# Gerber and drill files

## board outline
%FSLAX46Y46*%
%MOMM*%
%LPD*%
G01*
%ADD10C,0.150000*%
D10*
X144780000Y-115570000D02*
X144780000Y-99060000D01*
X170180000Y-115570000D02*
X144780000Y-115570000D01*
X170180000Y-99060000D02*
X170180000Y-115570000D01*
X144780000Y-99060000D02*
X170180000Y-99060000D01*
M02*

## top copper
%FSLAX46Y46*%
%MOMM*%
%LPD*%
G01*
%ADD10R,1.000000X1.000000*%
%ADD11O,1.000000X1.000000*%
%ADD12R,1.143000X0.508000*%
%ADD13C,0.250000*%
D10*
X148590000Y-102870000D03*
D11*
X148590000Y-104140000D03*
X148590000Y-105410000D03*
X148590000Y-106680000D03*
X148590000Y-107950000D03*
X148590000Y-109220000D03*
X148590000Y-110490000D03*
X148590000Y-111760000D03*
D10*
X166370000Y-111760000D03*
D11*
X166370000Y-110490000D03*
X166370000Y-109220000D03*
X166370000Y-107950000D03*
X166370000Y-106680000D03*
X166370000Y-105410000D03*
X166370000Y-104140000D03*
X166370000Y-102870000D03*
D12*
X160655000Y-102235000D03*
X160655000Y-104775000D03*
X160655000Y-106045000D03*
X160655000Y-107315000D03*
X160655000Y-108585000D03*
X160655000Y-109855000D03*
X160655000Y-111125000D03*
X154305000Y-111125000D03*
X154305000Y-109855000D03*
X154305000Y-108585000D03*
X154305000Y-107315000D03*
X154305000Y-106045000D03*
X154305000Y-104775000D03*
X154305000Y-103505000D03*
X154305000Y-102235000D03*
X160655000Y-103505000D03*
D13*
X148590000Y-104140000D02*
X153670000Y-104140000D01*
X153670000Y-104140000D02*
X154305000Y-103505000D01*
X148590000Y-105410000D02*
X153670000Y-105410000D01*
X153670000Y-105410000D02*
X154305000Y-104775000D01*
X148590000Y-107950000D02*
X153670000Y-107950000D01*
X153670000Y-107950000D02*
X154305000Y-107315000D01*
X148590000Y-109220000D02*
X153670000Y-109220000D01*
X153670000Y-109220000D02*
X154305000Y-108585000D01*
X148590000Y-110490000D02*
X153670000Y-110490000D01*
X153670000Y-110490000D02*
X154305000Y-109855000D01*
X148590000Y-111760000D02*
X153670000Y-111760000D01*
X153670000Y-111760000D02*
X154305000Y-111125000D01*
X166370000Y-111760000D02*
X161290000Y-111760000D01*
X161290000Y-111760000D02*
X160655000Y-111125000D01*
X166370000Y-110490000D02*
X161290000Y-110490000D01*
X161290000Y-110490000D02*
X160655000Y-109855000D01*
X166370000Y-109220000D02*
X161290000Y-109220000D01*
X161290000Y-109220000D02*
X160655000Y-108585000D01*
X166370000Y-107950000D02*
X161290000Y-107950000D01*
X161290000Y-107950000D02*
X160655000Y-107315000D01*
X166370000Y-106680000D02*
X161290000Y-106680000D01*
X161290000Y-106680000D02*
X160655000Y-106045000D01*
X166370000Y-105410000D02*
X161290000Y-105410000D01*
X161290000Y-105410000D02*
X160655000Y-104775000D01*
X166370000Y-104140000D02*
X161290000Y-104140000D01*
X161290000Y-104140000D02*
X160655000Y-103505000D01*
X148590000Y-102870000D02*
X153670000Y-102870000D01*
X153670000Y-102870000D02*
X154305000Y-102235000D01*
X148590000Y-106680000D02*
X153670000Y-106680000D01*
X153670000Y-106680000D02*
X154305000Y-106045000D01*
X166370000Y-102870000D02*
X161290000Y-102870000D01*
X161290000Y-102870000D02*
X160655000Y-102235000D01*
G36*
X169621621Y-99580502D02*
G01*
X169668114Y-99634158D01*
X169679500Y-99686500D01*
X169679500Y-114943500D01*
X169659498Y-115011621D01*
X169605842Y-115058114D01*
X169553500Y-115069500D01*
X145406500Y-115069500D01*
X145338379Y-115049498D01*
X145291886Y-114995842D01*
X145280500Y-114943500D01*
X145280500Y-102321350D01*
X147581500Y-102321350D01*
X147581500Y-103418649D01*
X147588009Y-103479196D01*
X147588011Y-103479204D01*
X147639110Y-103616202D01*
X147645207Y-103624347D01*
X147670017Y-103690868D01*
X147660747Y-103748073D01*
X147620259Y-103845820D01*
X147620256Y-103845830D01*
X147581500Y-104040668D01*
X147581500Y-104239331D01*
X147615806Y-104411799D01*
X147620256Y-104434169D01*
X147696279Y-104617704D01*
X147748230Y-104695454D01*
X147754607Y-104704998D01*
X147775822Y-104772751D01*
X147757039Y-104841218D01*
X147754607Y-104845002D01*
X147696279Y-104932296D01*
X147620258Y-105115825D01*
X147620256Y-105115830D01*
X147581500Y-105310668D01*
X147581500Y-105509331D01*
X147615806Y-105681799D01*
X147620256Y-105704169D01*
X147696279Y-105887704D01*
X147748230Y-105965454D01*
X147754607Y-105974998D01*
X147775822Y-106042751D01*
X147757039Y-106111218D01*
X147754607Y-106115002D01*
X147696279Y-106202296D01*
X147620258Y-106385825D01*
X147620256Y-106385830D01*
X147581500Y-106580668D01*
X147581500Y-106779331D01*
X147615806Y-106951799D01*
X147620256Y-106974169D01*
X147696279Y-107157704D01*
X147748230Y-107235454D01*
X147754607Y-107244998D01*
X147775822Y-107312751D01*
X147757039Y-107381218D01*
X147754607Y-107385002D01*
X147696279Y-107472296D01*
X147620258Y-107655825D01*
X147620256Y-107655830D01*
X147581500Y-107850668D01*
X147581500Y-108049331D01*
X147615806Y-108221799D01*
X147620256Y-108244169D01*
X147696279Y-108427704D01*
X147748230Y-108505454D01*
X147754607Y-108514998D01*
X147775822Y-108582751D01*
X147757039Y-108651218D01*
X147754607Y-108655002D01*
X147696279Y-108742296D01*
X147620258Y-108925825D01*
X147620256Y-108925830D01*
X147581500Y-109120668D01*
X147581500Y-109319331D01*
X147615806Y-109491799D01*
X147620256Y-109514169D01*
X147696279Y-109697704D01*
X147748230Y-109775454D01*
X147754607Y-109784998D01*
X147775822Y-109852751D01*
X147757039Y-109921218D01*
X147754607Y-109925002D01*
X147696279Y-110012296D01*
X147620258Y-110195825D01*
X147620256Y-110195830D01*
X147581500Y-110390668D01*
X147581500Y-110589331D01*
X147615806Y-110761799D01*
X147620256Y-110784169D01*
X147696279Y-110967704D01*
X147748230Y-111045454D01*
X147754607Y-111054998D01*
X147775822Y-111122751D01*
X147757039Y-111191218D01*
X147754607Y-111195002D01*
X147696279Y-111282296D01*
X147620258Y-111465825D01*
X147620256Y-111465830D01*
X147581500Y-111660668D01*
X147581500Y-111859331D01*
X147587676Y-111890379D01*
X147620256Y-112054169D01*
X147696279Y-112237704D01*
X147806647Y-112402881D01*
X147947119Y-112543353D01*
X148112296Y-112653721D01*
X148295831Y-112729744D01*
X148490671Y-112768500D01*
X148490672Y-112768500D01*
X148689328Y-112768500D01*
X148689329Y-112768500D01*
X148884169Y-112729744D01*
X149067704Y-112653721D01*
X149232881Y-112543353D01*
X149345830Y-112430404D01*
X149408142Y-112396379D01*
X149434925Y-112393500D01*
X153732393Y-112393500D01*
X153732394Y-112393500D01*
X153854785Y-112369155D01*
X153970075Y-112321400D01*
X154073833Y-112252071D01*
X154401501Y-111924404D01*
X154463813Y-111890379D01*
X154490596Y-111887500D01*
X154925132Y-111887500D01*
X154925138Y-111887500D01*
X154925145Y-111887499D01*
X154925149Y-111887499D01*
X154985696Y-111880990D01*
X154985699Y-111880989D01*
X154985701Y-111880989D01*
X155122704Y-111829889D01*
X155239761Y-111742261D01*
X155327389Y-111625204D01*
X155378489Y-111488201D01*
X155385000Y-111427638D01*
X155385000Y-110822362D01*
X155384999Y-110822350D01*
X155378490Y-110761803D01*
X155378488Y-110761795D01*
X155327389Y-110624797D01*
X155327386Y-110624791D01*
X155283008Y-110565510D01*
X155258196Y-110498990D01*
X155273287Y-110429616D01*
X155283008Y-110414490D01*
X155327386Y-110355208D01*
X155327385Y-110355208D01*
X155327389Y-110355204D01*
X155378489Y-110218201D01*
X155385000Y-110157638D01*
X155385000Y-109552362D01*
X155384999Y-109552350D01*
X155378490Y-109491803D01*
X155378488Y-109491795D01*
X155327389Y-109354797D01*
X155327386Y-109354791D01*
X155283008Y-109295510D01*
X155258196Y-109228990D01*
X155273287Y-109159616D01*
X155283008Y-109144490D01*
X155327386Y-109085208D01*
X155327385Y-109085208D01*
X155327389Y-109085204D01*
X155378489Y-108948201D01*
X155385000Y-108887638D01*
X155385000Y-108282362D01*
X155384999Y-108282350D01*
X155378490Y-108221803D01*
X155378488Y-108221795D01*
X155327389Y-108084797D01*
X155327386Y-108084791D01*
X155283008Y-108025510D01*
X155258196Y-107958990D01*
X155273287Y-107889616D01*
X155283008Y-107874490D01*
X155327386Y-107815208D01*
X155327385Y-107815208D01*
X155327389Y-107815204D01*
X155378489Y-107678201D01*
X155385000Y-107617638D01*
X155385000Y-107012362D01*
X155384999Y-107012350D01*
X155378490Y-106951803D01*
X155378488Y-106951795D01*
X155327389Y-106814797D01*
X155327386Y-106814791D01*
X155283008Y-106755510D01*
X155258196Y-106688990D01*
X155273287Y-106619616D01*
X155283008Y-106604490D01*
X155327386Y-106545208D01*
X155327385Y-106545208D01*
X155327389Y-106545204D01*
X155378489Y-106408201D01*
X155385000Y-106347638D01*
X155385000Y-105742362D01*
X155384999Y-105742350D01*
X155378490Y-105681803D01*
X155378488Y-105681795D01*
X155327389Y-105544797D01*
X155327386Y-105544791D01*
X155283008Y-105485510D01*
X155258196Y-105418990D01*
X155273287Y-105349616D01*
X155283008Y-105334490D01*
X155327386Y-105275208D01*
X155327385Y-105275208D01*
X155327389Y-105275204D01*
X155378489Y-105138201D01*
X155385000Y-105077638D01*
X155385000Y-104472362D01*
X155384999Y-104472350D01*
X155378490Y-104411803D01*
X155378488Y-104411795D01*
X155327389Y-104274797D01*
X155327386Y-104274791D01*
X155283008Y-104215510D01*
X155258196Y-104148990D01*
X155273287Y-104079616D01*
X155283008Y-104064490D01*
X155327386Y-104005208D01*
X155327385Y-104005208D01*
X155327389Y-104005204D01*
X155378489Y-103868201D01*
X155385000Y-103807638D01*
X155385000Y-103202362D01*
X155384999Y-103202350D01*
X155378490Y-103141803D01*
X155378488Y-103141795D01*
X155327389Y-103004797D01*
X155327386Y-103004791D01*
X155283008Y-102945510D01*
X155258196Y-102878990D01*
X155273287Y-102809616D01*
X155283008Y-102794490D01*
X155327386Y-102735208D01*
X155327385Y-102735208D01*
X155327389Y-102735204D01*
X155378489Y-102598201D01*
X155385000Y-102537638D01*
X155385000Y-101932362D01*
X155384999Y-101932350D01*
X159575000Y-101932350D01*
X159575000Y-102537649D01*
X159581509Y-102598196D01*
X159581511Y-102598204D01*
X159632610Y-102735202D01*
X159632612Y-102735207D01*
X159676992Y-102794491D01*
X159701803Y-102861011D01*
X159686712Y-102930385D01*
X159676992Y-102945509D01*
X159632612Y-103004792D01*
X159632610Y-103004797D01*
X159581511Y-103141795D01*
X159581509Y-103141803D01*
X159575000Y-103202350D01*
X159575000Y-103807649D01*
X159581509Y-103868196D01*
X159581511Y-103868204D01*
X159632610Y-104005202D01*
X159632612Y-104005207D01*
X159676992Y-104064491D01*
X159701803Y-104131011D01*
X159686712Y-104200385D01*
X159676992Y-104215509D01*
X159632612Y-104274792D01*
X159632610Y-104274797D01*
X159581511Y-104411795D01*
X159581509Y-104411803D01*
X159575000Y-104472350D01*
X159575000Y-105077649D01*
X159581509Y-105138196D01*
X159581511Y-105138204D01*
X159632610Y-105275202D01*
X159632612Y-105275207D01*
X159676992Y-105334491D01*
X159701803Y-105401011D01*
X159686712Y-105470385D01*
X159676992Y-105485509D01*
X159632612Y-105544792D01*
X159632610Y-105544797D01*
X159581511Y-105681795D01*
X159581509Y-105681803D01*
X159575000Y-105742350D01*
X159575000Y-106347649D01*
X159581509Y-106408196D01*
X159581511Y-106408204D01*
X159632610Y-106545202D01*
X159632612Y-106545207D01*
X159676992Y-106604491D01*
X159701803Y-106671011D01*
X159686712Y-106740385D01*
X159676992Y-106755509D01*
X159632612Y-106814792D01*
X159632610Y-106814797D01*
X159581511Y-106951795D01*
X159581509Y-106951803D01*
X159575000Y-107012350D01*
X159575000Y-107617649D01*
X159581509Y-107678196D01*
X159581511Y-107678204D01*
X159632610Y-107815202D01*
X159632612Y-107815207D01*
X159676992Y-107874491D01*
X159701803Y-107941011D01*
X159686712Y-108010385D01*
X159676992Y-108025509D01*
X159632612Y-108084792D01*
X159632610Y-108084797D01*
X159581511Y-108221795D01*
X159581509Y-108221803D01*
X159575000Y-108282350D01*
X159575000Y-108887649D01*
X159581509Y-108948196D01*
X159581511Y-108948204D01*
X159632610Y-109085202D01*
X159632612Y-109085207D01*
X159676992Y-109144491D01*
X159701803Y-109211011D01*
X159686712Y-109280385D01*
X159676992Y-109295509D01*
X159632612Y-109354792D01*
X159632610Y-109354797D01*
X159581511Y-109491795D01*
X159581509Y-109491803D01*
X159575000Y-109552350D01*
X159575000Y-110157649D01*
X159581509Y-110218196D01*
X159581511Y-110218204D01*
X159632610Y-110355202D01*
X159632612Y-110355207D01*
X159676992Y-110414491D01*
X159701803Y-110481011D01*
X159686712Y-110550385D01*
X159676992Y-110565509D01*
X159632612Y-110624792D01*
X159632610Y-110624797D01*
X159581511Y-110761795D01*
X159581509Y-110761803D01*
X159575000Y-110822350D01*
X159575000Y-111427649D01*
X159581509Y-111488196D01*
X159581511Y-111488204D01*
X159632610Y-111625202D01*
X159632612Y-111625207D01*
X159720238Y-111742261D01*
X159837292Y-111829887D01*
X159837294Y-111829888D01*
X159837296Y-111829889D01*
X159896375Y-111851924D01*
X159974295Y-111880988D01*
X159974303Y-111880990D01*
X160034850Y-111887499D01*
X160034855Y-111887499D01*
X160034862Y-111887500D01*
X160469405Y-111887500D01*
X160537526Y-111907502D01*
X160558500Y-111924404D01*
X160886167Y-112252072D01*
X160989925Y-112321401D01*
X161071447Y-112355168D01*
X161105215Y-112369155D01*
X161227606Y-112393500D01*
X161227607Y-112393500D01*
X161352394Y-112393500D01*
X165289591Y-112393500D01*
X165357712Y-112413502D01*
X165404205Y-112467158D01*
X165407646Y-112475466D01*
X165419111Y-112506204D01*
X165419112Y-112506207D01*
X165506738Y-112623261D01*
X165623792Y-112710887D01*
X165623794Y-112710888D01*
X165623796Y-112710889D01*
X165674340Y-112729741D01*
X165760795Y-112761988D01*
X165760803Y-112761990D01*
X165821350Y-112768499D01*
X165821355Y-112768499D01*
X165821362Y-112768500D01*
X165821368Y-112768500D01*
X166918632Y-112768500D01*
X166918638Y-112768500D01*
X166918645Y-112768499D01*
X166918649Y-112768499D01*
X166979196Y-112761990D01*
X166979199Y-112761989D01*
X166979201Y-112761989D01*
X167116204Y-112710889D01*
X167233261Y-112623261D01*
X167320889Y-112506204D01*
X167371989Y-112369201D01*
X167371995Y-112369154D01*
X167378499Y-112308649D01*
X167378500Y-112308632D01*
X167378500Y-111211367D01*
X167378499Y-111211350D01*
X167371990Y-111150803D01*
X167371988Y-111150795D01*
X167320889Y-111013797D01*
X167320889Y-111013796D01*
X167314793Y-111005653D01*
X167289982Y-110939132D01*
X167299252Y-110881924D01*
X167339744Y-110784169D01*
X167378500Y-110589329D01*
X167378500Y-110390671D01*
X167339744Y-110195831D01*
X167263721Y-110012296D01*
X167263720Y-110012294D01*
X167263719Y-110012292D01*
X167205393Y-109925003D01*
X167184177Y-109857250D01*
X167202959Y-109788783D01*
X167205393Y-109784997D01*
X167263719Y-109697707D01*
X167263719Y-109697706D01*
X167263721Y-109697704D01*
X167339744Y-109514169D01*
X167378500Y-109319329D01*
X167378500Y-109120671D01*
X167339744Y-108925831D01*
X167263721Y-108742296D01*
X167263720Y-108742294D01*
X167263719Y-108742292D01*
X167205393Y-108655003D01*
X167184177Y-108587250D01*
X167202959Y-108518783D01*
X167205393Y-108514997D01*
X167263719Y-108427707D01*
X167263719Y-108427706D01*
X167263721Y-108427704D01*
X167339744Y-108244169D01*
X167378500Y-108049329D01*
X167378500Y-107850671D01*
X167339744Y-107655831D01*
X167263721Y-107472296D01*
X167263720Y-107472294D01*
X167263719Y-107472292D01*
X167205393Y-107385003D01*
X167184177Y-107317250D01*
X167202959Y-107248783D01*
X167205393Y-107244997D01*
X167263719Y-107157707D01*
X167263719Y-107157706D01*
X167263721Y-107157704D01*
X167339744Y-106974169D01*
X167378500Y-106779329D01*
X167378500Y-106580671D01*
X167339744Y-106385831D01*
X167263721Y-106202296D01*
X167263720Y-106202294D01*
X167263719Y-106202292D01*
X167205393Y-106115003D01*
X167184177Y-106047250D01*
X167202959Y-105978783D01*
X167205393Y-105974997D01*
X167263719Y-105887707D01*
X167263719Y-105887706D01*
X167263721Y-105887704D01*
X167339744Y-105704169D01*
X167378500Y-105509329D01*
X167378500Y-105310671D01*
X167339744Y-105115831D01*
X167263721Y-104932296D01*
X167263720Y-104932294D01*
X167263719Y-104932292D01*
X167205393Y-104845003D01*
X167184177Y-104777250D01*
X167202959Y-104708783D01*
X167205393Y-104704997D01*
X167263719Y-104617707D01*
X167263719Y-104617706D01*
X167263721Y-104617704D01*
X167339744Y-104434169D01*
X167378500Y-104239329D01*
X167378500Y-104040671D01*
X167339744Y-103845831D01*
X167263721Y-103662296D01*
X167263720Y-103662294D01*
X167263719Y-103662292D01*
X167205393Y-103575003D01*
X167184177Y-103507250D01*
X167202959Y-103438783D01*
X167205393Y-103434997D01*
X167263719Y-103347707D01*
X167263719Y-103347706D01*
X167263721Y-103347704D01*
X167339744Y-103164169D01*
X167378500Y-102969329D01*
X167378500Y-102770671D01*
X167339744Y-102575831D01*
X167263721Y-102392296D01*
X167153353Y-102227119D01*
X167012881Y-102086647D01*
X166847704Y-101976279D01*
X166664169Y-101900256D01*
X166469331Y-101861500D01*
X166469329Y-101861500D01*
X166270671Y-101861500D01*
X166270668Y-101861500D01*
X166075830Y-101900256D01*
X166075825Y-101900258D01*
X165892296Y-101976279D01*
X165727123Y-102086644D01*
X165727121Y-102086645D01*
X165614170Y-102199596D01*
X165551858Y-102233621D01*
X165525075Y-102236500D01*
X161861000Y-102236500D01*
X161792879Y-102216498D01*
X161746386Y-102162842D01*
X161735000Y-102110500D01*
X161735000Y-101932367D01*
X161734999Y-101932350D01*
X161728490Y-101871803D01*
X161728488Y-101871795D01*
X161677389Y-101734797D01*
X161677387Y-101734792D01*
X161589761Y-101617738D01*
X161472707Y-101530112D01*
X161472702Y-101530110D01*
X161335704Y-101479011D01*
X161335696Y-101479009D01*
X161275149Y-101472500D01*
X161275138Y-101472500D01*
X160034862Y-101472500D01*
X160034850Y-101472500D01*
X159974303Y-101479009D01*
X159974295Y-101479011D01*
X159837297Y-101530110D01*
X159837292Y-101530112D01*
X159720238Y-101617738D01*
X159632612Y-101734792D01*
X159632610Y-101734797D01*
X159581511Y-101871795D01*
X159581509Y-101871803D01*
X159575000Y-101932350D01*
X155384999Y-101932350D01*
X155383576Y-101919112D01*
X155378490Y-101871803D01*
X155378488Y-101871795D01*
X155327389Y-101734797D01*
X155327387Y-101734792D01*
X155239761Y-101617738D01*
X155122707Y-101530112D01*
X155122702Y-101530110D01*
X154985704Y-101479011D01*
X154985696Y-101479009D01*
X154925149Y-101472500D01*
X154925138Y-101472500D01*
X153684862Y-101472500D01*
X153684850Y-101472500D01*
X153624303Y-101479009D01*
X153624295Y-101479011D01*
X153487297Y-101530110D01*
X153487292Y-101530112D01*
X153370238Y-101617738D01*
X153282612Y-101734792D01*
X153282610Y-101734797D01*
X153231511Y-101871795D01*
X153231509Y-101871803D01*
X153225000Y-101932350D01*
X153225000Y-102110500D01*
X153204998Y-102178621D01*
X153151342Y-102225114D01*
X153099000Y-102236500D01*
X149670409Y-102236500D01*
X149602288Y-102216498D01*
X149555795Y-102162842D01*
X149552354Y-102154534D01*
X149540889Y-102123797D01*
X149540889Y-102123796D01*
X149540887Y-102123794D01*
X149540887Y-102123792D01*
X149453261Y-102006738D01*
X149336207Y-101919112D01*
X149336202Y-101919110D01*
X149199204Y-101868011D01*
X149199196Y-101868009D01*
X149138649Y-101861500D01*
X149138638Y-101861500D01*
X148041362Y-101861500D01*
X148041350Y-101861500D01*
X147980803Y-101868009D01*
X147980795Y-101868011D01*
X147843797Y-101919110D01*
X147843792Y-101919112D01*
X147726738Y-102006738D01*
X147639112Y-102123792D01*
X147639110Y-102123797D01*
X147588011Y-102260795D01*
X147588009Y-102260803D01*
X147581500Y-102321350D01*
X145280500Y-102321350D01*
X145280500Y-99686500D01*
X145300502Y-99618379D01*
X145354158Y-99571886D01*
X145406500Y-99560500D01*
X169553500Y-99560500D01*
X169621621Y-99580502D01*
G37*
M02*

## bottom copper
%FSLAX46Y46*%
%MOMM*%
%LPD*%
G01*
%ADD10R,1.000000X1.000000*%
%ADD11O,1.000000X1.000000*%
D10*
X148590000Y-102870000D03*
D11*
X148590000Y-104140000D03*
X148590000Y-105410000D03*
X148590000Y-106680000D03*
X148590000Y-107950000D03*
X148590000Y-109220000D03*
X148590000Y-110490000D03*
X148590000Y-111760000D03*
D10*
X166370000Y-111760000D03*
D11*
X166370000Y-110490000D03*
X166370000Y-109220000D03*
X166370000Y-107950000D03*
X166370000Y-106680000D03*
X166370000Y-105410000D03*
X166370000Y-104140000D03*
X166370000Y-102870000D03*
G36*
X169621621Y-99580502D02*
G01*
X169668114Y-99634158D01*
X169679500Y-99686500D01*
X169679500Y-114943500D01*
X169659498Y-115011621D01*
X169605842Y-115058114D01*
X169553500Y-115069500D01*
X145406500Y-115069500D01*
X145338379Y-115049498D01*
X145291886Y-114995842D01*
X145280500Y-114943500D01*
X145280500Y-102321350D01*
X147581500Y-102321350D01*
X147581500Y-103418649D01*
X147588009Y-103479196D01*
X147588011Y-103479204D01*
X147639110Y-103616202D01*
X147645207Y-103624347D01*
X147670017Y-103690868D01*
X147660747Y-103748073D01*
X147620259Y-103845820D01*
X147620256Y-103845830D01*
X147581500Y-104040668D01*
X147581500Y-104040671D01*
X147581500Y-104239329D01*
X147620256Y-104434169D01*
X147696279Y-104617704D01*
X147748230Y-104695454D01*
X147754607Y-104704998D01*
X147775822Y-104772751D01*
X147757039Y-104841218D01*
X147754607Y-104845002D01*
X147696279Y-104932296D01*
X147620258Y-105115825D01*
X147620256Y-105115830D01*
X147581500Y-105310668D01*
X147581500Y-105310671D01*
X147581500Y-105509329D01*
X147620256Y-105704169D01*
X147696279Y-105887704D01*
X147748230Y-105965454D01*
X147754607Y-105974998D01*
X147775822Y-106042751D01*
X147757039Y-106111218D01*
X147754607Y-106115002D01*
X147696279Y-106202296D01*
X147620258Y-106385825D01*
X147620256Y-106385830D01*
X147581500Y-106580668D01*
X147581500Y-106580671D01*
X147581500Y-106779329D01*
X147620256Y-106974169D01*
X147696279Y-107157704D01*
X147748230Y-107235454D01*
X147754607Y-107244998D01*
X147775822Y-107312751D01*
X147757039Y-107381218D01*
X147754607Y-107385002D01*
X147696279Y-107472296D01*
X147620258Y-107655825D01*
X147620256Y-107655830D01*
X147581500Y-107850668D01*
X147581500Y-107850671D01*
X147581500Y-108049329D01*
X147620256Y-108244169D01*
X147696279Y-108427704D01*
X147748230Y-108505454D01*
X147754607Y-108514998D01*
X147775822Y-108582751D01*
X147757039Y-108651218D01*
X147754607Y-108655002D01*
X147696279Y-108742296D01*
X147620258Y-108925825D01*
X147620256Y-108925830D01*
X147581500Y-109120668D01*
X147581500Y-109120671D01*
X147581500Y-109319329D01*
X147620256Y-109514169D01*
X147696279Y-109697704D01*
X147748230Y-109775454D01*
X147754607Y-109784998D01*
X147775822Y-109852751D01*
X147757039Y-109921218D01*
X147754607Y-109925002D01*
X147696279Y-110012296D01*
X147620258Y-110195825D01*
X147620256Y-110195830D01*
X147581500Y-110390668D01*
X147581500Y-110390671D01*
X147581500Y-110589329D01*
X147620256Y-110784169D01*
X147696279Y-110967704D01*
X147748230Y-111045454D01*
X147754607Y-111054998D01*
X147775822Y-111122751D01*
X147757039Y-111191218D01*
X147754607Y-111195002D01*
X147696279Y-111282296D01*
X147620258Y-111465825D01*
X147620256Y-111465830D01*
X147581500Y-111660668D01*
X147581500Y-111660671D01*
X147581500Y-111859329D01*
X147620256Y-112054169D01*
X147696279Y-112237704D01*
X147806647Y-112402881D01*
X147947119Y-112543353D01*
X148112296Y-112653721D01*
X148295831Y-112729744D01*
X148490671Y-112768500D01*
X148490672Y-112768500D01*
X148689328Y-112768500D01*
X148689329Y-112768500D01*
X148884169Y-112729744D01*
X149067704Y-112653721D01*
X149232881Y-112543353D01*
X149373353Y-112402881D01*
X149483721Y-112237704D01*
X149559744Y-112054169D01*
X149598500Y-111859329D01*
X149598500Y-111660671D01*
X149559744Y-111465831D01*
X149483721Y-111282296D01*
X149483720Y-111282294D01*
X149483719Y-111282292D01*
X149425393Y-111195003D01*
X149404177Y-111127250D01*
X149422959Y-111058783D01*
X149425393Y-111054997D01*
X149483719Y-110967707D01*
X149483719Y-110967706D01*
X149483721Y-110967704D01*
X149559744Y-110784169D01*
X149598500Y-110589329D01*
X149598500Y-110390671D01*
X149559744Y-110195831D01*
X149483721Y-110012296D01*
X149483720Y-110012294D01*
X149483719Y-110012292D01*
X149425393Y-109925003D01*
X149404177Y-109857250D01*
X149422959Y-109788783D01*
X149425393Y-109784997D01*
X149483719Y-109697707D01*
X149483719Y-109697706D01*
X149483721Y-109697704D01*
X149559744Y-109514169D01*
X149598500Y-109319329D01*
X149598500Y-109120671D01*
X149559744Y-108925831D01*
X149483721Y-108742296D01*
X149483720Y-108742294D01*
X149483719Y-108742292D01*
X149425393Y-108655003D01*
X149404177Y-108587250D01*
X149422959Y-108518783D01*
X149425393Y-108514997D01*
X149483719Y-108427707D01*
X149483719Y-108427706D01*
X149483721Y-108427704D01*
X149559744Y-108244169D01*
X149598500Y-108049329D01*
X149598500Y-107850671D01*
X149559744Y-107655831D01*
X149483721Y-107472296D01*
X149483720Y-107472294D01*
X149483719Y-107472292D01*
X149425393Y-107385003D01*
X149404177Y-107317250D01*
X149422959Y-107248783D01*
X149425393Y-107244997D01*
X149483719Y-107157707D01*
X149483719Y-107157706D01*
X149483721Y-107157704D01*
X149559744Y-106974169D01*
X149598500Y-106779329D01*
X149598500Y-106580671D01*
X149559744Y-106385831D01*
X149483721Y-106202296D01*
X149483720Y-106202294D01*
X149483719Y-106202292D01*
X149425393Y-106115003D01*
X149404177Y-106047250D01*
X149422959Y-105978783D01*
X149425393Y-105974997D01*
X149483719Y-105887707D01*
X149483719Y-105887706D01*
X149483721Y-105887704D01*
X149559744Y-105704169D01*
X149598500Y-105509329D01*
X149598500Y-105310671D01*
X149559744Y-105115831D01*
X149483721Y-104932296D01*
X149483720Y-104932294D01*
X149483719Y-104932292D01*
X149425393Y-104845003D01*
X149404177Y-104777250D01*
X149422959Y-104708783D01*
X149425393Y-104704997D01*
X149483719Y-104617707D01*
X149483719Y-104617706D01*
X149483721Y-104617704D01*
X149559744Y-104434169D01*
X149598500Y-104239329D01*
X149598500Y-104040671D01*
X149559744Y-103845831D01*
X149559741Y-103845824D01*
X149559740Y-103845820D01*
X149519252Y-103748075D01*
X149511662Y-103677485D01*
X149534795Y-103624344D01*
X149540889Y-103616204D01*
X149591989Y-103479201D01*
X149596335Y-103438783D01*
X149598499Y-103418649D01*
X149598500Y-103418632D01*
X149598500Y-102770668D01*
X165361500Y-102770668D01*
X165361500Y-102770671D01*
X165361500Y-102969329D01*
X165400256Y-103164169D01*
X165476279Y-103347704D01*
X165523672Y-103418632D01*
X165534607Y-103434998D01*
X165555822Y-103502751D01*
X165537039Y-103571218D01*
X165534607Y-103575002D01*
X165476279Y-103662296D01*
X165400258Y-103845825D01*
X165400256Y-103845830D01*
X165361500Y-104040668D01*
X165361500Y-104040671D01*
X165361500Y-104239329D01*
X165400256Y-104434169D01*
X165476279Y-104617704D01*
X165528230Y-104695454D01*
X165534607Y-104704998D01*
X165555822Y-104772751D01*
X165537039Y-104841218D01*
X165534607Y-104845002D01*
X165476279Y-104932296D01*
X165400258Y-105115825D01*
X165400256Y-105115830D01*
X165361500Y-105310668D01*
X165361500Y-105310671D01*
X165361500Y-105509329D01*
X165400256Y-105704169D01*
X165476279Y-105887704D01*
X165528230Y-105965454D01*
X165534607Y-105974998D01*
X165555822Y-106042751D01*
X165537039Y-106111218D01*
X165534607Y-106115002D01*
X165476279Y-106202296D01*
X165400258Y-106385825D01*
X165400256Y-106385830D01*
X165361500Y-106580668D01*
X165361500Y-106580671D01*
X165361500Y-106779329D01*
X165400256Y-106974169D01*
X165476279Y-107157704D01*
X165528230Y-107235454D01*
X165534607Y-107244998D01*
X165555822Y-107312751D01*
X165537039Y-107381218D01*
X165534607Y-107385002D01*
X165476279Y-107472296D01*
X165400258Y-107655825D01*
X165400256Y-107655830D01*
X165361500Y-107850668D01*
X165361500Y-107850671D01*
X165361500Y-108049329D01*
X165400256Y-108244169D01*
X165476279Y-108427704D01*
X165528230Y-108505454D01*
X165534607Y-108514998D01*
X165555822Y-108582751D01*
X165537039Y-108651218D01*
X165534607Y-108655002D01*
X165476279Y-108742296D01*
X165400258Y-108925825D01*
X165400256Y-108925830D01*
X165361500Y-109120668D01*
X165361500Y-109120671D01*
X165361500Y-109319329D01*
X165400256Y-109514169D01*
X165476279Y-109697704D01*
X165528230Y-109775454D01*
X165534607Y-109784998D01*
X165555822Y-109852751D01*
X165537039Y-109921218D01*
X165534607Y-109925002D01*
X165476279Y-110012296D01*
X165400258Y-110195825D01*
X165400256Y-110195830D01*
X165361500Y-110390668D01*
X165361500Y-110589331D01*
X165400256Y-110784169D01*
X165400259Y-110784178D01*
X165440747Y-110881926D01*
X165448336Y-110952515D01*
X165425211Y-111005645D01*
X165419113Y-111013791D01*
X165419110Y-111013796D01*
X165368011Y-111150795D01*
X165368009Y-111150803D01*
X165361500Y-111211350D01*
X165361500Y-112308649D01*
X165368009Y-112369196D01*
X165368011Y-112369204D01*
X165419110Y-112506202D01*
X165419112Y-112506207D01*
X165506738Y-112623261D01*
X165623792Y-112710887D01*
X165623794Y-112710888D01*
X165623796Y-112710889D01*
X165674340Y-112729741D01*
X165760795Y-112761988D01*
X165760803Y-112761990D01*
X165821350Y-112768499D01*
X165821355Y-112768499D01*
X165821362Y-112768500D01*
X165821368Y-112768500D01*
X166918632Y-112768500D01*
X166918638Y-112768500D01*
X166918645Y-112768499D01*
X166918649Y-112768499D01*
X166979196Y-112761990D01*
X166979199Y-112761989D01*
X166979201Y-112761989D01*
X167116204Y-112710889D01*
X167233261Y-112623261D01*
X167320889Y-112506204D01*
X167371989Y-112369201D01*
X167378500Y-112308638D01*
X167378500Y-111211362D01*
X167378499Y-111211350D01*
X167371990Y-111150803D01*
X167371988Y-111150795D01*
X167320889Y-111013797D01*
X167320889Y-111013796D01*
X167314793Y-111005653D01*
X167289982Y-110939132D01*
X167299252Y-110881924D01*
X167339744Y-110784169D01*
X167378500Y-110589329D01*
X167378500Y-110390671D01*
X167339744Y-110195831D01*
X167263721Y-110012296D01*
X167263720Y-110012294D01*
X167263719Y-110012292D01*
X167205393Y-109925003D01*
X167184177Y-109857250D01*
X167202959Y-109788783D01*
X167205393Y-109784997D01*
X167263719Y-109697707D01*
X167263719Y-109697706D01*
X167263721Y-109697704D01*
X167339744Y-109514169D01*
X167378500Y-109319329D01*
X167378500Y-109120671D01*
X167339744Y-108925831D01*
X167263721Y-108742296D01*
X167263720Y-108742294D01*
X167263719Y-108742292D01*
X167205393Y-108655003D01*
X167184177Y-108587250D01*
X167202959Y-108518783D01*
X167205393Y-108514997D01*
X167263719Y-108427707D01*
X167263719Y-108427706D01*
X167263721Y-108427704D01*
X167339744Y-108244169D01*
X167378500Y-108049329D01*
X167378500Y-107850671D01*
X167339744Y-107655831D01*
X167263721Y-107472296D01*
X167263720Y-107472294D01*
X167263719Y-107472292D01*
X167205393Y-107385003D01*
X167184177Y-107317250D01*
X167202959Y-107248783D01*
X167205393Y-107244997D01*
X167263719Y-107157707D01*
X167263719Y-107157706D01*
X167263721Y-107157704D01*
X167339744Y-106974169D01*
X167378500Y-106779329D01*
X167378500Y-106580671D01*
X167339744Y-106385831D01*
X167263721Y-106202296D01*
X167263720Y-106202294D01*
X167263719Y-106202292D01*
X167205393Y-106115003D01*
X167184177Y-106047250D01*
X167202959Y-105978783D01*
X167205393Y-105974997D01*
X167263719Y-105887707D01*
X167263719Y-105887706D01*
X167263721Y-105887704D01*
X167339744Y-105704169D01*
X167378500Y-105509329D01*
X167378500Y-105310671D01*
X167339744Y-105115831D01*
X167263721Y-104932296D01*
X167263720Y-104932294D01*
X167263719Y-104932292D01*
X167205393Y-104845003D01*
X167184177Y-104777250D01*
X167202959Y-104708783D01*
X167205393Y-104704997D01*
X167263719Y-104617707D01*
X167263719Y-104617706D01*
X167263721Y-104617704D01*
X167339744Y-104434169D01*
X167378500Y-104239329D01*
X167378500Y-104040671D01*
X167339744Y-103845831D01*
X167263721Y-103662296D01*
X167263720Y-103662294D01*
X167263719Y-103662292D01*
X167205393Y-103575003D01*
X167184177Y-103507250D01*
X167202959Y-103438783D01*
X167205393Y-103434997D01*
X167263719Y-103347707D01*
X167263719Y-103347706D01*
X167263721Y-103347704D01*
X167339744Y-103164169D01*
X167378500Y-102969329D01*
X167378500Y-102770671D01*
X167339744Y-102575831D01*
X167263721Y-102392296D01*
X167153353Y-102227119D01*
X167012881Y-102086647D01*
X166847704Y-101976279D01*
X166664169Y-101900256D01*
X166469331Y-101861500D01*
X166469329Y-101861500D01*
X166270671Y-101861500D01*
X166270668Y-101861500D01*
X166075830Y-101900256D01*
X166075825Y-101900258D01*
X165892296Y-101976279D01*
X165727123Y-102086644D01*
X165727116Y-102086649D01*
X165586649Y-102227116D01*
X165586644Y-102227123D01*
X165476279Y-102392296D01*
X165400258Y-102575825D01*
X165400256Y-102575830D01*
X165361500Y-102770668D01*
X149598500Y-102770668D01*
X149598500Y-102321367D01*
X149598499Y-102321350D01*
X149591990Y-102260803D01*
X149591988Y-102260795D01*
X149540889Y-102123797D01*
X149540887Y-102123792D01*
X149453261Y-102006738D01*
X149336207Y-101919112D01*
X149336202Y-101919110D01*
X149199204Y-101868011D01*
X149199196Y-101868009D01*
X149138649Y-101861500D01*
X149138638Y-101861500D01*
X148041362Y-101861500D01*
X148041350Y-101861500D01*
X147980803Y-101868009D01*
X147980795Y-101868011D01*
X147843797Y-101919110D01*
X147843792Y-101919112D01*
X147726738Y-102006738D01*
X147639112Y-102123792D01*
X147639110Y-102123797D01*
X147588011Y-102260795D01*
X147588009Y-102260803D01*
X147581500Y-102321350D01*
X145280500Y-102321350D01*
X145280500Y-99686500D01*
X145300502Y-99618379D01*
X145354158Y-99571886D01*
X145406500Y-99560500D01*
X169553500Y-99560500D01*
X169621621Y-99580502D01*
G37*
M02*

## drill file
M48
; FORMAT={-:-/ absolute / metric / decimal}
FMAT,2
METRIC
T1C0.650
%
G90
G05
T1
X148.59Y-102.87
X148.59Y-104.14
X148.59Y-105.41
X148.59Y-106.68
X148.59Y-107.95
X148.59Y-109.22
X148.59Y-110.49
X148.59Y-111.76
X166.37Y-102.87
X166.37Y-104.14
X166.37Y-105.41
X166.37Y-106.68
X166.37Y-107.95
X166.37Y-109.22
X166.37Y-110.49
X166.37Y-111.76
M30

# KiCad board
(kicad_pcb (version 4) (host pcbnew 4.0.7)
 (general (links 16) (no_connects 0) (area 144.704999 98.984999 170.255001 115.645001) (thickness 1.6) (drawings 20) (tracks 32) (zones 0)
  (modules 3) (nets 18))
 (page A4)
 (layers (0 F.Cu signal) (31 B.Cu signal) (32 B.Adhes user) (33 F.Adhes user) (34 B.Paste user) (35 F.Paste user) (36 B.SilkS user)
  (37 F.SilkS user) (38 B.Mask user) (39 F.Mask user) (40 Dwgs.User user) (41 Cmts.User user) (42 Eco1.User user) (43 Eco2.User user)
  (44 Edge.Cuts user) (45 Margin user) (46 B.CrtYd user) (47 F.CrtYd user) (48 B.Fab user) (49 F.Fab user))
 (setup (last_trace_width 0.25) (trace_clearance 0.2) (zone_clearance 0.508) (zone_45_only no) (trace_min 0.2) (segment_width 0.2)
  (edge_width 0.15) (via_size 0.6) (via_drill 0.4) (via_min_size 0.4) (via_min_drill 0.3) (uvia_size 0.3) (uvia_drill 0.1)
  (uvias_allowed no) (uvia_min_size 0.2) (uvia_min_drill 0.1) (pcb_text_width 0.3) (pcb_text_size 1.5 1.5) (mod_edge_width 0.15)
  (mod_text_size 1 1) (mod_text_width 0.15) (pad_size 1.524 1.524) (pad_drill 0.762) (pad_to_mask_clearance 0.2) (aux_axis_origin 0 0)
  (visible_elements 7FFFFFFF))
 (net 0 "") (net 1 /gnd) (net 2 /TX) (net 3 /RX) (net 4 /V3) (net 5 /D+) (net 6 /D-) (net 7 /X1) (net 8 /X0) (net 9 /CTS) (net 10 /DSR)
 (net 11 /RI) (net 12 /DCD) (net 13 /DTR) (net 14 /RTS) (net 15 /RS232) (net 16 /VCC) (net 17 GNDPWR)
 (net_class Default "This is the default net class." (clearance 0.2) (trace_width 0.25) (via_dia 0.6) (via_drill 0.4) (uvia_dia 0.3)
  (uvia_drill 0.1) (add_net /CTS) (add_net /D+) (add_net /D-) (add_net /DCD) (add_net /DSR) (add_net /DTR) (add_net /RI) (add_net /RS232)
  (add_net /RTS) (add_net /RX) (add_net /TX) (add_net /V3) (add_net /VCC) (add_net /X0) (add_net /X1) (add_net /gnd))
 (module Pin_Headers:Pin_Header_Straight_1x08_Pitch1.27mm (layer F.Cu) (at 148.59 102.87)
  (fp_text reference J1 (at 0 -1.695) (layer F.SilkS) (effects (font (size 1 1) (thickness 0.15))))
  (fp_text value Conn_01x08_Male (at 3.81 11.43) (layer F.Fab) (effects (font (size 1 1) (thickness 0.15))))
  (pad 1 thru_hole rect (at 0 0) (size 1 1) (drill 0.65) (layers *.Cu *.Mask) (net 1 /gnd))
  (pad 2 thru_hole oval (at 0 1.27) (size 1 1) (drill 0.65) (layers *.Cu *.Mask) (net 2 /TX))
  (pad 3 thru_hole oval (at 0 2.54) (size 1 1) (drill 0.65) (layers *.Cu *.Mask) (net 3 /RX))
  (pad 4 thru_hole oval (at 0 3.81) (size 1 1) (drill 0.65) (layers *.Cu *.Mask) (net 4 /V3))
  (pad 5 thru_hole oval (at 0 5.08) (size 1 1) (drill 0.65) (layers *.Cu *.Mask) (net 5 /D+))
  (pad 6 thru_hole oval (at 0 6.35) (size 1 1) (drill 0.65) (layers *.Cu *.Mask) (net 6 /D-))
  (pad 7 thru_hole oval (at 0 7.62) (size 1 1) (drill 0.65) (layers *.Cu *.Mask) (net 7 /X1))
  (pad 8 thru_hole oval (at 0 8.89) (size 1 1) (drill 0.65) (layers *.Cu *.Mask) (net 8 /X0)))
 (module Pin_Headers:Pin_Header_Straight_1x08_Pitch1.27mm (layer F.Cu) (at 166.37 111.76 180)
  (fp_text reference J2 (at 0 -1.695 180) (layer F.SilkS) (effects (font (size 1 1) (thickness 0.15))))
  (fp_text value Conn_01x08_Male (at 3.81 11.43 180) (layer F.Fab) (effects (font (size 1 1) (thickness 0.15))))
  (pad 1 thru_hole rect (at 0 0 180) (size 1 1) (drill 0.65) (layers *.Cu *.Mask) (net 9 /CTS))
  (pad 2 thru_hole oval (at 0 1.27 180) (size 1 1) (drill 0.65) (layers *.Cu *.Mask) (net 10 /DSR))
  (pad 3 thru_hole oval (at 0 2.54 180) (size 1 1) (drill 0.65) (layers *.Cu *.Mask) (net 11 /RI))
  (pad 4 thru_hole oval (at 0 3.81 180) (size 1 1) (drill 0.65) (layers *.Cu *.Mask) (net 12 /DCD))
  (pad 5 thru_hole oval (at 0 5.08 180) (size 1 1) (drill 0.65) (layers *.Cu *.Mask) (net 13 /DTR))
  (pad 6 thru_hole oval (at 0 6.35 180) (size 1 1) (drill 0.65) (layers *.Cu *.Mask) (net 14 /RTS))
  (pad 7 thru_hole oval (at 0 7.62 180) (size 1 1) (drill 0.65) (layers *.Cu *.Mask) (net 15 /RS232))
  (pad 8 thru_hole oval (at 0 8.89 180) (size 1 1) (drill 0.65) (layers *.Cu *.Mask) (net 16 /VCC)))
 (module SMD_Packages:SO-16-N (layer F.Cu) (at 157.48 106.68 270)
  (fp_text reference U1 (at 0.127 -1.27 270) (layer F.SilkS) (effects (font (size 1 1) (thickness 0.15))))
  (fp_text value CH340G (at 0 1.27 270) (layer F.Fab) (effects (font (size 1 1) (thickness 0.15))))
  (pad 16 smd rect (at -4.445 -3.175 270) (size 0.508 1.143) (layers F.Cu F.Paste F.Mask) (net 16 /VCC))
  (pad 14 smd rect (at -1.905 -3.175 270) (size 0.508 1.143) (layers F.Cu F.Paste F.Mask) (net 14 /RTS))
  (pad 13 smd rect (at -0.635 -3.175 270) (size 0.508 1.143) (layers F.Cu F.Paste F.Mask) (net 13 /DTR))
  (pad 12 smd rect (at 0.635 -3.175 270) (size 0.508 1.143) (layers F.Cu F.Paste F.Mask) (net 12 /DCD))
  (pad 11 smd rect (at 1.905 -3.175 270) (size 0.508 1.143) (layers F.Cu F.Paste F.Mask) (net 11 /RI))
  (pad 10 smd rect (at 3.175 -3.175 270) (size 0.508 1.143) (layers F.Cu F.Paste F.Mask) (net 10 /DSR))
  (pad 9 smd rect (at 4.445 -3.175 270) (size 0.508 1.143) (layers F.Cu F.Paste F.Mask) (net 9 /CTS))
  (pad 8 smd rect (at 4.445 3.175 270) (size 0.508 1.143) (layers F.Cu F.Paste F.Mask) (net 8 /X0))
  (pad 7 smd rect (at 3.175 3.175 270) (size 0.508 1.143) (layers F.Cu F.Paste F.Mask) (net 7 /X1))
  (pad 6 smd rect (at 1.905 3.175 270) (size 0.508 1.143) (layers F.Cu F.Paste F.Mask) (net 6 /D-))
  (pad 5 smd rect (at 0.635 3.175 270) (size 0.508 1.143) (layers F.Cu F.Paste F.Mask) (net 5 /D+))
  (pad 4 smd rect (at -0.635 3.175 270) (size 0.508 1.143) (layers F.Cu F.Paste F.Mask) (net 4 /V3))
  (pad 3 smd rect (at -1.905 3.175 270) (size 0.508 1.143) (layers F.Cu F.Paste F.Mask) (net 3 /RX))
  (pad 2 smd rect (at -3.175 3.175 270) (size 0.508 1.143) (layers F.Cu F.Paste F.Mask) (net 2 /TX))
  (pad 1 smd rect (at -4.445 3.175 270) (size 0.508 1.143) (layers F.Cu F.Paste F.Mask) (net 1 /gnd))
  (pad 15 smd rect (at -3.175 -3.175 270) (size 0.508 1.143) (layers F.Cu F.Paste F.Mask) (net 15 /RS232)))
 (gr_line (start 144.78 115.57) (end 144.78 99.06) (angle 90) (layer Edge.Cuts) (width 0.15))
 (gr_line (start 170.18 115.57) (end 144.78 115.57) (angle 90) (layer Edge.Cuts) (width 0.15))
 (gr_line (start 170.18 99.06) (end 170.18 115.57) (angle 90) (layer Edge.Cuts) (width 0.15))
 (gr_line (start 144.78 99.06) (end 170.18 99.06) (angle 90) (layer Edge.Cuts) (width 0.15))
 (segment (start 148.59 104.14) (end 153.67 104.14) (width 0.25) (layer F.Cu) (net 2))
 (segment (start 153.67 104.14) (end 154.305 103.505) (width 0.25) (layer F.Cu) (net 2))
 (segment (start 148.59 105.41) (end 153.67 105.41) (width 0.25) (layer F.Cu) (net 3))
 (segment (start 153.67 105.41) (end 154.305 104.775) (width 0.25) (layer F.Cu) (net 3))
 (segment (start 148.59 107.95) (end 153.67 107.95) (width 0.25) (layer F.Cu) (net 5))
 (segment (start 153.67 107.95) (end 154.305 107.315) (width 0.25) (layer F.Cu) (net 5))
 (segment (start 148.59 109.22) (end 153.67 109.22) (width 0.25) (layer F.Cu) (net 6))
 (segment (start 153.67 109.22) (end 154.305 108.585) (width 0.25) (layer F.Cu) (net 6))
 (segment (start 148.59 110.49) (end 153.67 110.49) (width 0.25) (layer F.Cu) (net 7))
 (segment (start 153.67 110.49) (end 154.305 109.855) (width 0.25) (layer F.Cu) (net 7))
 (segment (start 148.59 111.76) (end 153.67 111.76) (width 0.25) (layer F.Cu) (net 8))
 (segment (start 153.67 111.76) (end 154.305 111.125) (width 0.25) (layer F.Cu) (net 8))
 (segment (start 166.37 111.76) (end 161.29 111.76) (width 0.25) (layer F.Cu) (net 9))
 (segment (start 161.29 111.76) (end 160.655 111.125) (width 0.25) (layer F.Cu) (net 9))
 (segment (start 166.37 110.49) (end 161.29 110.49) (width 0.25) (layer F.Cu) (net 10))
 (segment (start 161.29 110.49) (end 160.655 109.855) (width 0.25) (layer F.Cu) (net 10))
 (segment (start 166.37 109.22) (end 161.29 109.22) (width 0.25) (layer F.Cu) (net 11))
 (segment (start 161.29 109.22) (end 160.655 108.585) (width 0.25) (layer F.Cu) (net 11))
 (segment (start 166.37 107.95) (end 161.29 107.95) (width 0.25) (layer F.Cu) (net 12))
 (segment (start 161.29 107.95) (end 160.655 107.315) (width 0.25) (layer F.Cu) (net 12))
 (segment (start 166.37 106.68) (end 161.29 106.68) (width 0.25) (layer F.Cu) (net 13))
 (segment (start 161.29 106.68) (end 160.655 106.045) (width 0.25) (layer F.Cu) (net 13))
 (segment (start 166.37 105.41) (end 161.29 105.41) (width 0.25) (layer F.Cu) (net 14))
 (segment (start 161.29 105.41) (end 160.655 104.775) (width 0.25) (layer F.Cu) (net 14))
 (segment (start 166.37 104.14) (end 161.29 104.14) (width 0.25) (layer F.Cu) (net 15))
 (segment (start 161.29 104.14) (end 160.655 103.505) (width 0.25) (layer F.Cu) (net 15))
 (segment (start 148.59 102.87) (end 153.67 102.87) (width 0.25) (layer F.Cu) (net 1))
 (segment (start 153.67 102.87) (end 154.305 102.235) (width 0.25) (layer F.Cu) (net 1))
 (segment (start 148.59 106.68) (end 153.67 106.68) (width 0.25) (layer F.Cu) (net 4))
 (segment (start 153.67 106.68) (end 154.305 106.045) (width 0.25) (layer F.Cu) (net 4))
 (segment (start 166.37 102.87) (end 161.29 102.87) (width 0.25) (layer F.Cu) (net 16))
 (segment (start 161.29 102.87) (end 160.655 102.235) (width 0.25) (layer F.Cu) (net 16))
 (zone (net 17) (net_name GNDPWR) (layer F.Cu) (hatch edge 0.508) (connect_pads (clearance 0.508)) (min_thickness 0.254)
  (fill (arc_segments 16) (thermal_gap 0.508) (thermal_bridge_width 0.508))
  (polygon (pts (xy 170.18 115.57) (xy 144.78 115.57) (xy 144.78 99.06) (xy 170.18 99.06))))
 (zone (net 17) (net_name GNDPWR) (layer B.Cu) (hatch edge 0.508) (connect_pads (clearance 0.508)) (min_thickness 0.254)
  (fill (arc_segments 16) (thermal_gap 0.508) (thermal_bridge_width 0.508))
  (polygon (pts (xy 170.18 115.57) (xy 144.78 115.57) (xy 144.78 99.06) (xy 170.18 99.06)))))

